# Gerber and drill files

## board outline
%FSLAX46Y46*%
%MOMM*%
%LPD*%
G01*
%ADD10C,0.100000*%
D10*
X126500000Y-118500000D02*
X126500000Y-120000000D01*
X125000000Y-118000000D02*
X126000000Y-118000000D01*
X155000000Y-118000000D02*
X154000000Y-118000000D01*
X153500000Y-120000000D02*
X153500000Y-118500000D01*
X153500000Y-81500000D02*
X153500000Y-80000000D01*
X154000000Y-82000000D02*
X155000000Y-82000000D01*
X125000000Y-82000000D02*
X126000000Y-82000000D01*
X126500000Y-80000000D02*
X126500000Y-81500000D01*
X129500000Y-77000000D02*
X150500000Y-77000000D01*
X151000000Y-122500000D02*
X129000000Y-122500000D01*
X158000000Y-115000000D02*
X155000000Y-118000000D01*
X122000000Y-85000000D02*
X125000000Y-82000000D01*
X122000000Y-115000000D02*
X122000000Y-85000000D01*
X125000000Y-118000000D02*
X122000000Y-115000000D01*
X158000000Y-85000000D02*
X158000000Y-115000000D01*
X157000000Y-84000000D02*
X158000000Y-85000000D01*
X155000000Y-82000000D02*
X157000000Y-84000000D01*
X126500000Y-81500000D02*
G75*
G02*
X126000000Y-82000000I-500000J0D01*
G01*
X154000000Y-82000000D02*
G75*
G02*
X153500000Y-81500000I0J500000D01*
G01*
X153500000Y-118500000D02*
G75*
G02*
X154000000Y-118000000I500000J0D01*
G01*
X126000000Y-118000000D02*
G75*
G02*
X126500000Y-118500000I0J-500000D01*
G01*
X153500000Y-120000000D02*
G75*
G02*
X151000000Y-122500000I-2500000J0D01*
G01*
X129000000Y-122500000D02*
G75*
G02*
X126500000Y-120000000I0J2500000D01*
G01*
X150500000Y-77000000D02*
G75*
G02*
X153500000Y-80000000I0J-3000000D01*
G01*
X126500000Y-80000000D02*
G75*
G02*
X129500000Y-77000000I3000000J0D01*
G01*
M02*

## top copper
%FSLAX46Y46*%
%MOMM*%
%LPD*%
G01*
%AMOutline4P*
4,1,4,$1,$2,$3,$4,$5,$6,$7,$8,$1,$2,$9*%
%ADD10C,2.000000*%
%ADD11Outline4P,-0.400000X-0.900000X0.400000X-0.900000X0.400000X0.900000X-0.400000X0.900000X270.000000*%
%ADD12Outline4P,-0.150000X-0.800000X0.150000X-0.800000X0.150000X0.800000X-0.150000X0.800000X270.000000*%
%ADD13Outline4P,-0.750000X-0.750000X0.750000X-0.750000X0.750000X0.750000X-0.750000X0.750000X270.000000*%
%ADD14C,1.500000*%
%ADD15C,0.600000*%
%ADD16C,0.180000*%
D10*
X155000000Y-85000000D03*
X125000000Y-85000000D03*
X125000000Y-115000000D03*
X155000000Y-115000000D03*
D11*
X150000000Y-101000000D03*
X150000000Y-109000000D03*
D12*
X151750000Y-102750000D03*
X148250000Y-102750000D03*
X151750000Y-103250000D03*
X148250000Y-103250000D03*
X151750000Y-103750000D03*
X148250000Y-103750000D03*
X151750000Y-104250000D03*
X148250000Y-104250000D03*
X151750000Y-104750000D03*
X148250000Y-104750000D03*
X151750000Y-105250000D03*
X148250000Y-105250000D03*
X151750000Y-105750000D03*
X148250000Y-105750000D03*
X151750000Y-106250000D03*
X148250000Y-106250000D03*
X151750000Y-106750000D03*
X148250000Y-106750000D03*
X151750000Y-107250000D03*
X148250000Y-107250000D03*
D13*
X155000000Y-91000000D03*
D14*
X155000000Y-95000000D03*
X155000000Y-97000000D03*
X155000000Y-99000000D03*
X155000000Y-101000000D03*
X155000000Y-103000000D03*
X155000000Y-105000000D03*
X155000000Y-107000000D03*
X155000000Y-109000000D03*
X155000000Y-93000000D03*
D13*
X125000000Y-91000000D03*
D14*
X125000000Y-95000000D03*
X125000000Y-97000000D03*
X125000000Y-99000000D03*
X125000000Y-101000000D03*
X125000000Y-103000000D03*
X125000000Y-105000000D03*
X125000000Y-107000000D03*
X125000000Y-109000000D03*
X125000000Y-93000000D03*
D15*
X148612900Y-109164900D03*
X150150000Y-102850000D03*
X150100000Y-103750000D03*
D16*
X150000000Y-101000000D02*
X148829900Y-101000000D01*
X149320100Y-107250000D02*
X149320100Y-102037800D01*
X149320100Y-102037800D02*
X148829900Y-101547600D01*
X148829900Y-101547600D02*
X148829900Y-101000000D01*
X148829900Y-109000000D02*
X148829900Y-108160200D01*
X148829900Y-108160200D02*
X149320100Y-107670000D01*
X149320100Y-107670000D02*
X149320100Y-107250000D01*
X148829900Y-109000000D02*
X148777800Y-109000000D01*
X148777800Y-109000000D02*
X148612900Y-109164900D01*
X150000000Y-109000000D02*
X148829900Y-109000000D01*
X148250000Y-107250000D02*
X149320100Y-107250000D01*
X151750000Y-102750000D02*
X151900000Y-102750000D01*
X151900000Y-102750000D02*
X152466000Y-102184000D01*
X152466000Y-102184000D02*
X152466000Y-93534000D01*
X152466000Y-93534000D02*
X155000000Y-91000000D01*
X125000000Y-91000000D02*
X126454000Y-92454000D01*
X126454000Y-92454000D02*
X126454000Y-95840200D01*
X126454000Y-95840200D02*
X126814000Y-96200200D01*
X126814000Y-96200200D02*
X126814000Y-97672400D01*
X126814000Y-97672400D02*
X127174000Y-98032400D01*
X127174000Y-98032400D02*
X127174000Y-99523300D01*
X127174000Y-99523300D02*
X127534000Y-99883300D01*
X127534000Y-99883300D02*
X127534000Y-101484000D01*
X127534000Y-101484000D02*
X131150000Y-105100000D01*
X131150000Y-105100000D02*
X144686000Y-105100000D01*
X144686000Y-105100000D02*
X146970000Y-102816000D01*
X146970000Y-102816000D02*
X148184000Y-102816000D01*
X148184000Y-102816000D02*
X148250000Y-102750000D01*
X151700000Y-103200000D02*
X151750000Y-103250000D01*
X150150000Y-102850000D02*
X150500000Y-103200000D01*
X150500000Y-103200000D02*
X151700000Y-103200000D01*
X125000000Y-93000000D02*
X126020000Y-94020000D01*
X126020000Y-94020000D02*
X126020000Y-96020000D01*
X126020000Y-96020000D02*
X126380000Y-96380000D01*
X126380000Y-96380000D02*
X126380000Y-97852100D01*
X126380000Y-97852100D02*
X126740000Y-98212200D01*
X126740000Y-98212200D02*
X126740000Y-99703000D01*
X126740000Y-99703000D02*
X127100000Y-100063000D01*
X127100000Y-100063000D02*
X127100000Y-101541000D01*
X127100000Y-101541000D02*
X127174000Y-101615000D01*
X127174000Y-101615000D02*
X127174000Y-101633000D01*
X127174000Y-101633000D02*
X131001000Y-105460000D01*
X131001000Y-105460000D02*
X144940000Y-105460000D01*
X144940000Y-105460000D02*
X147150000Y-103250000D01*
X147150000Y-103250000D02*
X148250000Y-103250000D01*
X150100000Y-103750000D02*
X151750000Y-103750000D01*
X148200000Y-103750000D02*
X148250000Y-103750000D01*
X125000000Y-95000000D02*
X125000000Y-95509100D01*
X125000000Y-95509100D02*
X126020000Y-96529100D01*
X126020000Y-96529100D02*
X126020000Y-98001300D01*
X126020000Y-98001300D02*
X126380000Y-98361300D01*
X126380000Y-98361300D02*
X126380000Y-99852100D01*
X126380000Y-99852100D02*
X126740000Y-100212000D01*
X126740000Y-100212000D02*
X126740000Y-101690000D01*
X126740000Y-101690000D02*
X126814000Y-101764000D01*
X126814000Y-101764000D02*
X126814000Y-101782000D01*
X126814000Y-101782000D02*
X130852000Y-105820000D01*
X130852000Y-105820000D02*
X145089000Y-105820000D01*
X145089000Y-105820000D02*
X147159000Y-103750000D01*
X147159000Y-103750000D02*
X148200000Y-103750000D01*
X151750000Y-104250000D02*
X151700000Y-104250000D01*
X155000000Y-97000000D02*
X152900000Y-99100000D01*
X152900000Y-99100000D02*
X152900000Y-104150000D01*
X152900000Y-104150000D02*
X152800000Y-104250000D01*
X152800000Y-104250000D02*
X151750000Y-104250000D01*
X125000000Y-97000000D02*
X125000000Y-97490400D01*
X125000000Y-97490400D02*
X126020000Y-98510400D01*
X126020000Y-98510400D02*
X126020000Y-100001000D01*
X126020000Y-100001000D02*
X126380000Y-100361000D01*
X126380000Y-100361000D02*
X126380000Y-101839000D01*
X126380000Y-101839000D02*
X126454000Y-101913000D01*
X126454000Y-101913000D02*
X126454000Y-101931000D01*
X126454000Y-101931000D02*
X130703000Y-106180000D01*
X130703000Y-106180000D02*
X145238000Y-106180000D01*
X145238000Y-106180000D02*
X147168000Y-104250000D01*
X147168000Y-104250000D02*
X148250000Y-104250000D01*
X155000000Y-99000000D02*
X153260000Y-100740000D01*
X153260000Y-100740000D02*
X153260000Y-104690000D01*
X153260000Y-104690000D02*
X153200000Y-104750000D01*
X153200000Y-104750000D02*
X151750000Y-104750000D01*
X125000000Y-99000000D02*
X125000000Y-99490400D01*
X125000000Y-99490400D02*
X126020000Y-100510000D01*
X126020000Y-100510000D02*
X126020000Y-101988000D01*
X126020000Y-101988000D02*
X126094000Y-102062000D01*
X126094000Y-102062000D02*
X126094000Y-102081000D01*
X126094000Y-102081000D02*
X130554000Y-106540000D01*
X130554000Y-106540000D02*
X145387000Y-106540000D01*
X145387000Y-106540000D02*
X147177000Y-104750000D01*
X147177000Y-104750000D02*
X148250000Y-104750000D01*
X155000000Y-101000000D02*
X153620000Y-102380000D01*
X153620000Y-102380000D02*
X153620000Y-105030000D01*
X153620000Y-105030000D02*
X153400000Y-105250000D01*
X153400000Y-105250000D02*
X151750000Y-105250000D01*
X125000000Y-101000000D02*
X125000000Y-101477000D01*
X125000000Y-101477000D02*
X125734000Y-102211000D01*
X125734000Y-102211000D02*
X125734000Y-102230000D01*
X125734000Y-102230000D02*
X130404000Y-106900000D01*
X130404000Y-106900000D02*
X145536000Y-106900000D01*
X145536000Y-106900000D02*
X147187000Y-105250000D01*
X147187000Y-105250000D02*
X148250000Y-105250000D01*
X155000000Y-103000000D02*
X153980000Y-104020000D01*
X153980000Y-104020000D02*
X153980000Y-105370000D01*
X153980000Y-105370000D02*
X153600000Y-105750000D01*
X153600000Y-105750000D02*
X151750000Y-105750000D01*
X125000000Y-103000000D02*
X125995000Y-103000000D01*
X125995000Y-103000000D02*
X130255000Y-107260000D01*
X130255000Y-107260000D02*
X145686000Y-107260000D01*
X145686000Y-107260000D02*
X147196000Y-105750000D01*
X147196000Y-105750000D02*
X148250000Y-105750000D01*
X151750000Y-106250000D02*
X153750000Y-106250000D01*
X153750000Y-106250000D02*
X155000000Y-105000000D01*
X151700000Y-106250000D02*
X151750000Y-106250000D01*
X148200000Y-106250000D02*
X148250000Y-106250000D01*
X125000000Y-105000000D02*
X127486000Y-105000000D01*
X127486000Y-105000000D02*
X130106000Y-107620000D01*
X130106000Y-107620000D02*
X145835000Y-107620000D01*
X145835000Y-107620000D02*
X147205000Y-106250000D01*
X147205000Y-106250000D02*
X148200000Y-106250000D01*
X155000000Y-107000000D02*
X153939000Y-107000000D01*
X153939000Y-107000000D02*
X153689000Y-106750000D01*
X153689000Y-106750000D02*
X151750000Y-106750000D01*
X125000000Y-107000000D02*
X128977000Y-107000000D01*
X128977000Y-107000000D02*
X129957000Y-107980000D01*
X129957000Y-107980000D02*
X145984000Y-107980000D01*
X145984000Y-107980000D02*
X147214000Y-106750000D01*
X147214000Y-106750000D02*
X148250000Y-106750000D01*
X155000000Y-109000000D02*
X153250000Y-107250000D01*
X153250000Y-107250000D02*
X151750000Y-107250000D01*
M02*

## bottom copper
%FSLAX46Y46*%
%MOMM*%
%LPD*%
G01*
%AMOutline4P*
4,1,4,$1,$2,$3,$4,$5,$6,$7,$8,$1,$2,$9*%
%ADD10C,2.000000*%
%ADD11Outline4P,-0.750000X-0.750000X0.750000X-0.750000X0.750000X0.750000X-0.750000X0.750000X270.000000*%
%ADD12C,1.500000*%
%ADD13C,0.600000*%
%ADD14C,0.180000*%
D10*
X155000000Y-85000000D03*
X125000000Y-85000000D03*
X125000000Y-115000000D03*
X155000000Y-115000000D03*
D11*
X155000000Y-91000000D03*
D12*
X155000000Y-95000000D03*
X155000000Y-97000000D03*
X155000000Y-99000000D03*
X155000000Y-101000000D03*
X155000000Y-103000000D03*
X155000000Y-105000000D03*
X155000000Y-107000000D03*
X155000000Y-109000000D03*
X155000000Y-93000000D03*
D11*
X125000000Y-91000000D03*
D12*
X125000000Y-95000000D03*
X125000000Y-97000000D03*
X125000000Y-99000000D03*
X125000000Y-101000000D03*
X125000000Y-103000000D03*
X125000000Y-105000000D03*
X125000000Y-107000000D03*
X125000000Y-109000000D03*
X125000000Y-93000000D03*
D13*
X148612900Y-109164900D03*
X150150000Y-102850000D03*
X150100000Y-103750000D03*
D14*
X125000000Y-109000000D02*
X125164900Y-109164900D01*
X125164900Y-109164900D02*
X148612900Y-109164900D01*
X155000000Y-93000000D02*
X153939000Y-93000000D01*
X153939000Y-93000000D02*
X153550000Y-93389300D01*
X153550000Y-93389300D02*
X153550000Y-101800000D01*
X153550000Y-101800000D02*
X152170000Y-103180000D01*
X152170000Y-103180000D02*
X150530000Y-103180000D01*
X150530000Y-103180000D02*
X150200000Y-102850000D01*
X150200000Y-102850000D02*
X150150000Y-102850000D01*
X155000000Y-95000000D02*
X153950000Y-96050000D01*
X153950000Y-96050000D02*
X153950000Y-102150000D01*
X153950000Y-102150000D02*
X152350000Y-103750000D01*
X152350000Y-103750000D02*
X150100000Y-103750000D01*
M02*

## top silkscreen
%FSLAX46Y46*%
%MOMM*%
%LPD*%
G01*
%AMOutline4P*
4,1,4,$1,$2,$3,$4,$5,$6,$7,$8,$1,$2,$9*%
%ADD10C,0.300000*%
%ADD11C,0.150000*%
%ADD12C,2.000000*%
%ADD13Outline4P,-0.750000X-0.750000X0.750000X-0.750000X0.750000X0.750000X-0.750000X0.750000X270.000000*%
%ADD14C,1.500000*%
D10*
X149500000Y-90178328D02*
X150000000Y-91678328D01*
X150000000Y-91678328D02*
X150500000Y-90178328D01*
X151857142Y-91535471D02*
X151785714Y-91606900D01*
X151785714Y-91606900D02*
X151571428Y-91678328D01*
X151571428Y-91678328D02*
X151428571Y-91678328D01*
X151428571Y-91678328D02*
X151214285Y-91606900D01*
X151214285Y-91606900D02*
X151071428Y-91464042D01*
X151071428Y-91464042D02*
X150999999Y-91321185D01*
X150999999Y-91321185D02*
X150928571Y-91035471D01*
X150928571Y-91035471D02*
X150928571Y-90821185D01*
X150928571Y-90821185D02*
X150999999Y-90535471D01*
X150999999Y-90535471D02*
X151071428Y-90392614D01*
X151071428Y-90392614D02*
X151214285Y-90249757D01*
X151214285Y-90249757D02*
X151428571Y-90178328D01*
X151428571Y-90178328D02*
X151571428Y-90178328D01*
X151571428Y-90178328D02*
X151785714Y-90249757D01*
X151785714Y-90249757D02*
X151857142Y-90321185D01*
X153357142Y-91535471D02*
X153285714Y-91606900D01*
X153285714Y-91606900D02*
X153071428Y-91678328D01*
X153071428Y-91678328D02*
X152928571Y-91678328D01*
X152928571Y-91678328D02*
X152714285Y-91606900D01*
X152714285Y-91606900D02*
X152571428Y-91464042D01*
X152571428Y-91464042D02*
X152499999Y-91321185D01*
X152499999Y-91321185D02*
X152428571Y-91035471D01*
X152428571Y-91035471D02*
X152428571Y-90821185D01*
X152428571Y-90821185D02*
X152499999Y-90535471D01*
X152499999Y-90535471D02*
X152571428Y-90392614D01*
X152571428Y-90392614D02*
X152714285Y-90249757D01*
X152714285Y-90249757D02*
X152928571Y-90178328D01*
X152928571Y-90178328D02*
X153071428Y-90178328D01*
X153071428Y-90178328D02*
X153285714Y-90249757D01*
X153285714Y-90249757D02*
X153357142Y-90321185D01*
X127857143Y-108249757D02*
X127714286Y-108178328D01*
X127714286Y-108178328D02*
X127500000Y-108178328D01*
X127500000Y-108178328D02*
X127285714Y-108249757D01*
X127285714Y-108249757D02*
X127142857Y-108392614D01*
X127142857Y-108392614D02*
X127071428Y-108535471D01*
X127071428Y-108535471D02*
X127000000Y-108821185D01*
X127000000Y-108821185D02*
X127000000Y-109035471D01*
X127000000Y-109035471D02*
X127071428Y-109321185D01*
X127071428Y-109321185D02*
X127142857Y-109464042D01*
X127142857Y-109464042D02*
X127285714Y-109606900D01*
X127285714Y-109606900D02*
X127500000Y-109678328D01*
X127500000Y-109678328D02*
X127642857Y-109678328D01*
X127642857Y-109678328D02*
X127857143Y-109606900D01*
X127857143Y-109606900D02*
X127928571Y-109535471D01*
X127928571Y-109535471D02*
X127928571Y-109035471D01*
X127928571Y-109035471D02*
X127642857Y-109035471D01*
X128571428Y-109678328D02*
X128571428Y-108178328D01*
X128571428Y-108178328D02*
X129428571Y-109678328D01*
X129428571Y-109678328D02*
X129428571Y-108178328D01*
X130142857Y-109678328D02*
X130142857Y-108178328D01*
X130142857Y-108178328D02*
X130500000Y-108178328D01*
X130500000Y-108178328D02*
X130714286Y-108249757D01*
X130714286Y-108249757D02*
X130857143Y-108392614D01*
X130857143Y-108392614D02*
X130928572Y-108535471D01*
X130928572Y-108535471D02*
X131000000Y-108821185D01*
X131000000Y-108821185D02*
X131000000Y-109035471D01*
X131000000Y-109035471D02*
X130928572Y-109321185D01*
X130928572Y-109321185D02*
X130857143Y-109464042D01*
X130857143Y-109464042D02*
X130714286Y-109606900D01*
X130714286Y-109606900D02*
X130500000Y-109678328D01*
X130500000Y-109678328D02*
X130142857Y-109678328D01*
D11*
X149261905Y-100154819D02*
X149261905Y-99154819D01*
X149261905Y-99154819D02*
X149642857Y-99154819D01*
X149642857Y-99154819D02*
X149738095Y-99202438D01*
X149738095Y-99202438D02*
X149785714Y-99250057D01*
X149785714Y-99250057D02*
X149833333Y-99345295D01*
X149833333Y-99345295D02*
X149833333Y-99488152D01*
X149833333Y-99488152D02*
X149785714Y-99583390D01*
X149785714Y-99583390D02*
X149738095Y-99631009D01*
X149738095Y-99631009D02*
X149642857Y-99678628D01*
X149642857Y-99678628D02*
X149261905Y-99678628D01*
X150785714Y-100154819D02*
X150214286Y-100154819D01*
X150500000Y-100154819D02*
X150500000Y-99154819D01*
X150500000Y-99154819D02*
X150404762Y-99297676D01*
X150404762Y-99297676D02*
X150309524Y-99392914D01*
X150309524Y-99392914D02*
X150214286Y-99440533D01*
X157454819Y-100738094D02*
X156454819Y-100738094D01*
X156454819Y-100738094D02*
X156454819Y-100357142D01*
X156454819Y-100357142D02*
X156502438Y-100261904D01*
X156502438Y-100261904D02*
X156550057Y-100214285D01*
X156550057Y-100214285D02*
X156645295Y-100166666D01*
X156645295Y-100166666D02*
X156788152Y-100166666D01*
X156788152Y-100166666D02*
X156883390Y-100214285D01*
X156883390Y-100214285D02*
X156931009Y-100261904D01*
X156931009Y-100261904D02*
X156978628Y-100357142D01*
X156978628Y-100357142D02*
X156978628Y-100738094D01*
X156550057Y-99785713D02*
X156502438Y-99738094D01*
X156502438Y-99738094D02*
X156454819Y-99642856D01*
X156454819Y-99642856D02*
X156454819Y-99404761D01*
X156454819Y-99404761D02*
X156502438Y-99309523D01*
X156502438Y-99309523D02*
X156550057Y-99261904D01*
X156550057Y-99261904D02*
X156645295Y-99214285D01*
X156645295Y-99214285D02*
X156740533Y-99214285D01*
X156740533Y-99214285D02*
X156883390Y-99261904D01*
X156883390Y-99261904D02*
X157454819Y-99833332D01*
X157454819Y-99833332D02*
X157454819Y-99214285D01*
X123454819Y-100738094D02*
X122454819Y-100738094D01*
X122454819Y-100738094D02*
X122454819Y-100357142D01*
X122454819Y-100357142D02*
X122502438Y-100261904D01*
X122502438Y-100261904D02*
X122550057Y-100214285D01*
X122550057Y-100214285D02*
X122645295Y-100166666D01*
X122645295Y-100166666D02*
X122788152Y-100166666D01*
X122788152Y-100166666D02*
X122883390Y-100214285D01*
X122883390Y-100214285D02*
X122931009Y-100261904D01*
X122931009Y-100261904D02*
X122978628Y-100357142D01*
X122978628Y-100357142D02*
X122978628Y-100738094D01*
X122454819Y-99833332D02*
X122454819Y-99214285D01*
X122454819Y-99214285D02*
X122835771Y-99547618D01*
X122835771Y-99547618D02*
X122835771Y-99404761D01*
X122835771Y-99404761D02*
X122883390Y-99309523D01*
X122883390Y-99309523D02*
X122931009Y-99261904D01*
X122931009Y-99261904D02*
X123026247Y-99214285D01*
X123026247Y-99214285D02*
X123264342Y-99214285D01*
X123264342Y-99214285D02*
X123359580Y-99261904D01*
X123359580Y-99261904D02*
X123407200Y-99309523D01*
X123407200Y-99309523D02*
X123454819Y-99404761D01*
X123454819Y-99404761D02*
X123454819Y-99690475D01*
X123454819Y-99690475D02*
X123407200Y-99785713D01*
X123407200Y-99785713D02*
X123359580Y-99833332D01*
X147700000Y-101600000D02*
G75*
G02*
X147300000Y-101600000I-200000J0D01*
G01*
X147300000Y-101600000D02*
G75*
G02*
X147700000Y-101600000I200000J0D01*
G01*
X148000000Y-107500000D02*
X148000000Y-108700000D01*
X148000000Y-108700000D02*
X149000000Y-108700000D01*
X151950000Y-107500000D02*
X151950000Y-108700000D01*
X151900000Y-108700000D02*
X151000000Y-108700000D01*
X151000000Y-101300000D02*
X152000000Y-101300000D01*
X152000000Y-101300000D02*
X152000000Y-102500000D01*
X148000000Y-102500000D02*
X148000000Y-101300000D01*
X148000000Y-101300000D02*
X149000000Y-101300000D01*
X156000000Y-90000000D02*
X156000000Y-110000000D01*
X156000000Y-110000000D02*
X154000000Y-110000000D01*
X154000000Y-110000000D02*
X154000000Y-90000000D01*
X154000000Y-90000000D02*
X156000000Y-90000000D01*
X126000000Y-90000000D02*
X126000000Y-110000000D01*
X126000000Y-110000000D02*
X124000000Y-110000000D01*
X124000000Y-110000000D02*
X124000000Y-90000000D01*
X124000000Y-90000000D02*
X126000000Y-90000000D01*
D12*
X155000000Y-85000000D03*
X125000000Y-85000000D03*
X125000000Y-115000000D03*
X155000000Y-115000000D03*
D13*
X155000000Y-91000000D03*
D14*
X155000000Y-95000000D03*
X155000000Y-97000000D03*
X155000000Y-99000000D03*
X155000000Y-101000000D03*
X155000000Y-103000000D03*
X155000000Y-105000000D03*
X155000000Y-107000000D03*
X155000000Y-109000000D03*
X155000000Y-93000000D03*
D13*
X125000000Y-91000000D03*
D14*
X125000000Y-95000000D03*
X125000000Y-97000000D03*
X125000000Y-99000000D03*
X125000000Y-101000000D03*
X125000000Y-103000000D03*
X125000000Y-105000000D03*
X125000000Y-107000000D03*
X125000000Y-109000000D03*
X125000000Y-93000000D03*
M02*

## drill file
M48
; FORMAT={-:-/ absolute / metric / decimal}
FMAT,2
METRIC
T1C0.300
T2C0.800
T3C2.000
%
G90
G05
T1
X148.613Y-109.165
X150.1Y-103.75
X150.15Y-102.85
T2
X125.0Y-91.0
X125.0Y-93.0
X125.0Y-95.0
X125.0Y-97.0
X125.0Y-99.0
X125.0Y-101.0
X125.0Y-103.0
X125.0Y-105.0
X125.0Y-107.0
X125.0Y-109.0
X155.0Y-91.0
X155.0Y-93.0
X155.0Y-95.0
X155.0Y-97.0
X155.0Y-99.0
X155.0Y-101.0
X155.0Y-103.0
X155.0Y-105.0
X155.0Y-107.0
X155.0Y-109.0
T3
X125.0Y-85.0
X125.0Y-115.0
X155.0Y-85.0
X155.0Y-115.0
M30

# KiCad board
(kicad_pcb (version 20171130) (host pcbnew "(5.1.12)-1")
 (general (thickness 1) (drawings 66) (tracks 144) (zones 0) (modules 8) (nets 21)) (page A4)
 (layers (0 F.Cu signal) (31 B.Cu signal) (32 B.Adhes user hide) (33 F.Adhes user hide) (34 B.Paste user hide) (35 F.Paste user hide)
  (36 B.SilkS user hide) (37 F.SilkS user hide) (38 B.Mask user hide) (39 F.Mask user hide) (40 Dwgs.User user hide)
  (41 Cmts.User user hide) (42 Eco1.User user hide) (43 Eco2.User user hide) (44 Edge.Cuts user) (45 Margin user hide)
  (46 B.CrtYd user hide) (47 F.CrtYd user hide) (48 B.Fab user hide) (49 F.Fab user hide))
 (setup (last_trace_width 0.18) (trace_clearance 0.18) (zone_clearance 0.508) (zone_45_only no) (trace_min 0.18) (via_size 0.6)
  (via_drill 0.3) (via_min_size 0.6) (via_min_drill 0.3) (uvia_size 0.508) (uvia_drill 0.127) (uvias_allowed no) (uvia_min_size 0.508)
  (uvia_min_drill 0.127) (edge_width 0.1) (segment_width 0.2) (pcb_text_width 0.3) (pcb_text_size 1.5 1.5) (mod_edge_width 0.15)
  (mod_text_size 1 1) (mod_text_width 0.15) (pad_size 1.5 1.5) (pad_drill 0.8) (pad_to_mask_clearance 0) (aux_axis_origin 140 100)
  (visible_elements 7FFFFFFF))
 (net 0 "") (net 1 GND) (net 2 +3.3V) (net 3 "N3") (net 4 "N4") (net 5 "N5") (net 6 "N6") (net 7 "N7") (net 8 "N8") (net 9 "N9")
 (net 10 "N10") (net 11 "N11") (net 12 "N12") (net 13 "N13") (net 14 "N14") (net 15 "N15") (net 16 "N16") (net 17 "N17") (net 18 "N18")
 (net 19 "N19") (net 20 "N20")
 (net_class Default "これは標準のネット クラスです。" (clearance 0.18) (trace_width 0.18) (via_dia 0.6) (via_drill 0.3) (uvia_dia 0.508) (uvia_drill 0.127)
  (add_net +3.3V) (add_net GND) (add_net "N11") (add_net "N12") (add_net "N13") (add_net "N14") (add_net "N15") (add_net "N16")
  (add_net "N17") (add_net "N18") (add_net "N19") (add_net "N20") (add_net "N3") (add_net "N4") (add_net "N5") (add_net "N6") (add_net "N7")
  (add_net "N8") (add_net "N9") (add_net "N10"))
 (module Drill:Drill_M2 (layer F.Cu) (at 155 85)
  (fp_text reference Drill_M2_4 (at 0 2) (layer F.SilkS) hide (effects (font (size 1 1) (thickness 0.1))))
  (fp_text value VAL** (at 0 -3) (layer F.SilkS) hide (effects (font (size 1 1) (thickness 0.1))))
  (pad "" thru_hole circle (at 0 0) (size 2 2) (drill 2) (layers *.Cu *.Mask F.SilkS)))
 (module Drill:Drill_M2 (layer F.Cu) (at 125 85)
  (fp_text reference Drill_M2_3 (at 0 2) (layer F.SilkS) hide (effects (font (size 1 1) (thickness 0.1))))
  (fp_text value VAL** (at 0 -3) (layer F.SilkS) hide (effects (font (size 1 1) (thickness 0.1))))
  (pad "" thru_hole circle (at 0 0) (size 2 2) (drill 2) (layers *.Cu *.Mask F.SilkS)))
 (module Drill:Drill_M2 (layer F.Cu) (at 125 115)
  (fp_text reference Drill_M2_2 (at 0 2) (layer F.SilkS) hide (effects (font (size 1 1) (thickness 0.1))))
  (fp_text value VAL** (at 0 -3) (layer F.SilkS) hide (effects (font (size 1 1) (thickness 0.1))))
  (pad "" thru_hole circle (at 0 0) (size 2 2) (drill 2) (layers *.Cu *.Mask F.SilkS)))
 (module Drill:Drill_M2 (layer F.Cu) (at 155 115)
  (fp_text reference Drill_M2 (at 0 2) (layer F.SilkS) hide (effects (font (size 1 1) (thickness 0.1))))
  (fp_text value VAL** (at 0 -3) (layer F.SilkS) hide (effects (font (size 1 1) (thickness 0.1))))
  (pad "" thru_hole circle (at 0 0) (size 2 2) (drill 2) (layers *.Cu *.Mask F.SilkS)))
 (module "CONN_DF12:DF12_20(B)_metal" (layer F.Cu) (at 150 105)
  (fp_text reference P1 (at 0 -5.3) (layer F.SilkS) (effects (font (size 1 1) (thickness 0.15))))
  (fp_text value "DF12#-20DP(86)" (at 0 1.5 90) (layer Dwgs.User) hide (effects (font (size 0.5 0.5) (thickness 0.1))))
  (fp_circle (center -2.5 -3.4) (end -2.5 -3.2) (layer F.SilkS) (width 0.15))
  (fp_line (start -2 2.5) (end -2 3.7) (layer F.SilkS) (width 0.15))
  (fp_line (start -2 3.7) (end -1 3.7) (layer F.SilkS) (width 0.15))
  (fp_line (start 1.95 2.5) (end 1.95 3.7) (layer F.SilkS) (width 0.15))
  (fp_line (start 1.9 3.7) (end 1 3.7) (layer F.SilkS) (width 0.15))
  (fp_line (start 1 -3.7) (end 2 -3.7) (layer F.SilkS) (width 0.15))
  (fp_line (start 2 -3.7) (end 2 -2.5) (layer F.SilkS) (width 0.15))
  (fp_line (start -2 -2.5) (end -2 -3.7) (layer F.SilkS) (width 0.15))
  (fp_line (start -2 -3.7) (end -1 -3.7) (layer F.SilkS) (width 0.15))
  (pad 21 smd trapezoid (at 0 -4 270) (size 0.8 1.8) (layers F.Cu F.Paste F.Mask) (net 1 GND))
  (pad 22 smd trapezoid (at 0 4 270) (size 0.8 1.8) (layers F.Cu F.Paste F.Mask) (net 1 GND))
  (pad 1 smd trapezoid (at 1.75 -2.25 270) (size 0.3 1.6) (layers F.Cu F.Paste F.Mask) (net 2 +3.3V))
  (pad 2 smd trapezoid (at -1.75 -2.25 270) (size 0.3 1.6) (layers F.Cu F.Paste F.Mask) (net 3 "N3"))
  (pad 3 smd trapezoid (at 1.75 -1.75 270) (size 0.3 1.6) (layers F.Cu F.Paste F.Mask) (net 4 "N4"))
  (pad 4 smd trapezoid (at -1.75 -1.75 270) (size 0.3 1.6) (layers F.Cu F.Paste F.Mask) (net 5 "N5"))
  (pad 5 smd trapezoid (at 1.75 -1.25 270) (size 0.3 1.6) (layers F.Cu F.Paste F.Mask) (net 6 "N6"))
  (pad 6 smd trapezoid (at -1.75 -1.25 270) (size 0.3 1.6) (layers F.Cu F.Paste F.Mask) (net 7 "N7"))
  (pad 7 smd trapezoid (at 1.75 -0.75 270) (size 0.3 1.6) (layers F.Cu F.Paste F.Mask) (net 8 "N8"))
  (pad 8 smd trapezoid (at -1.75 -0.75 270) (size 0.3 1.6) (layers F.Cu F.Paste F.Mask) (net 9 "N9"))
  (pad 9 smd trapezoid (at 1.75 -0.25 270) (size 0.3 1.6) (layers F.Cu F.Paste F.Mask) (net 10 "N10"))
  (pad 10 smd trapezoid (at -1.75 -0.25 270) (size 0.3 1.6) (layers F.Cu F.Paste F.Mask) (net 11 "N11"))
  (pad 11 smd trapezoid (at 1.75 0.25 270) (size 0.3 1.6) (layers F.Cu F.Paste F.Mask) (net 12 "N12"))
  (pad 12 smd trapezoid (at -1.75 0.25 270) (size 0.3 1.6) (layers F.Cu F.Paste F.Mask) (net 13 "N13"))
  (pad 13 smd trapezoid (at 1.75 0.75 270) (size 0.3 1.6) (layers F.Cu F.Paste F.Mask) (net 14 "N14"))
  (pad 14 smd trapezoid (at -1.75 0.75 270) (size 0.3 1.6) (layers F.Cu F.Paste F.Mask) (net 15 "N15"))
  (pad 15 smd trapezoid (at 1.75 1.25 270) (size 0.3 1.6) (layers F.Cu F.Paste F.Mask) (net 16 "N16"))
  (pad 16 smd trapezoid (at -1.75 1.25 270) (size 0.3 1.6) (layers F.Cu F.Paste F.Mask) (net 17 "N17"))
  (pad 17 smd trapezoid (at 1.75 1.75 270) (size 0.3 1.6) (layers F.Cu F.Paste F.Mask) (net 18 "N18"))
  (pad 18 smd trapezoid (at -1.75 1.75 270) (size 0.3 1.6) (layers F.Cu F.Paste F.Mask) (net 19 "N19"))
  (pad 19 smd trapezoid (at 1.75 2.25 270) (size 0.3 1.6) (layers F.Cu F.Paste F.Mask) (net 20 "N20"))
  (pad 20 smd trapezoid (at -1.75 2.25 270) (size 0.3 1.6) (layers F.Cu F.Paste F.Mask) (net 1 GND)))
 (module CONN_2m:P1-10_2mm (layer F.Cu) (at 155 100 270)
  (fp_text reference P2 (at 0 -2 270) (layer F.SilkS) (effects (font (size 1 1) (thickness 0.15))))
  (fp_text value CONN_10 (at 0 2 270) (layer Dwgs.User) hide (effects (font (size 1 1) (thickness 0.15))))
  (fp_line (start -10 -1) (end 10 -1) (layer F.SilkS) (width 0.15))
  (fp_line (start 10 -1) (end 10 1) (layer F.SilkS) (width 0.15))
  (fp_line (start 10 1) (end -10 1) (layer F.SilkS) (width 0.15))
  (fp_line (start -10 1) (end -10 -1) (layer F.SilkS) (width 0.15))
  (pad 1 thru_hole trapezoid (at -9 0 270) (size 1.5 1.5) (drill 0.8) (layers *.Cu *.Mask F.SilkS) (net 2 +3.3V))
  (pad 3 thru_hole circle (at -5 0 270) (size 1.5 1.5) (drill 0.8) (layers *.Cu *.Mask F.SilkS) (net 6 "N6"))
  (pad 4 thru_hole circle (at -3 0 270) (size 1.5 1.5) (drill 0.8) (layers *.Cu *.Mask F.SilkS) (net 8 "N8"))
  (pad 5 thru_hole circle (at -1 0 270) (size 1.5 1.5) (drill 0.8) (layers *.Cu *.Mask F.SilkS) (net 10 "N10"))
  (pad 6 thru_hole circle (at 1 0 270) (size 1.5 1.5) (drill 0.8) (layers *.Cu *.Mask F.SilkS) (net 12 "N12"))
  (pad 7 thru_hole circle (at 3 0 270) (size 1.5 1.5) (drill 0.8) (layers *.Cu *.Mask F.SilkS) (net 14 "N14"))
  (pad 8 thru_hole circle (at 5 0 270) (size 1.5 1.5) (drill 0.8) (layers *.Cu *.Mask F.SilkS) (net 16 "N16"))
  (pad 9 thru_hole circle (at 7 0 270) (size 1.5 1.5) (drill 0.8) (layers *.Cu *.Mask F.SilkS) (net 18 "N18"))
  (pad 10 thru_hole circle (at 9 0 270) (size 1.5 1.5) (drill 0.8) (layers *.Cu *.Mask F.SilkS) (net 20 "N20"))
  (pad 2 thru_hole circle (at -7 0 270) (size 1.5 1.5) (drill 0.8) (layers *.Cu *.Mask F.SilkS) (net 4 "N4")))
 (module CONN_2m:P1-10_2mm (layer F.Cu) (at 125 100 270)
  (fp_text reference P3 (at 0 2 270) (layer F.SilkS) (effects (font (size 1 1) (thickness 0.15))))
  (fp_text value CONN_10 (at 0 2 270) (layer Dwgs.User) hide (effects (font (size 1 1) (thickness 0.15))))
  (fp_line (start -10 -1) (end 10 -1) (layer F.SilkS) (width 0.15))
  (fp_line (start 10 -1) (end 10 1) (layer F.SilkS) (width 0.15))
  (fp_line (start 10 1) (end -10 1) (layer F.SilkS) (width 0.15))
  (fp_line (start -10 1) (end -10 -1) (layer F.SilkS) (width 0.15))
  (pad 1 thru_hole trapezoid (at -9 0 270) (size 1.5 1.5) (drill 0.8) (layers *.Cu *.Mask F.SilkS) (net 3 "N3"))
  (pad 3 thru_hole circle (at -5 0 270) (size 1.5 1.5) (drill 0.8) (layers *.Cu *.Mask F.SilkS) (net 7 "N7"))
  (pad 4 thru_hole circle (at -3 0 270) (size 1.5 1.5) (drill 0.8) (layers *.Cu *.Mask F.SilkS) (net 9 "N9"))
  (pad 5 thru_hole circle (at -1 0 270) (size 1.5 1.5) (drill 0.8) (layers *.Cu *.Mask F.SilkS) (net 11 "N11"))
  (pad 6 thru_hole circle (at 1 0 270) (size 1.5 1.5) (drill 0.8) (layers *.Cu *.Mask F.SilkS) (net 13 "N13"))
  (pad 7 thru_hole circle (at 3 0 270) (size 1.5 1.5) (drill 0.8) (layers *.Cu *.Mask F.SilkS) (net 15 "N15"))
  (pad 8 thru_hole circle (at 5 0 270) (size 1.5 1.5) (drill 0.8) (layers *.Cu *.Mask F.SilkS) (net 17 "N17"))
  (pad 9 thru_hole circle (at 7 0 270) (size 1.5 1.5) (drill 0.8) (layers *.Cu *.Mask F.SilkS) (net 19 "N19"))
  (pad 10 thru_hole circle (at 9 0 270) (size 1.5 1.5) (drill 0.8) (layers *.Cu *.Mask F.SilkS) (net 1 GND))
  (pad 2 thru_hole circle (at -7 0 270) (size 1.5 1.5) (drill 0.8) (layers *.Cu *.Mask F.SilkS) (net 5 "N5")))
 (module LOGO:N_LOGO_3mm (layer B.Cu) (at 140 95)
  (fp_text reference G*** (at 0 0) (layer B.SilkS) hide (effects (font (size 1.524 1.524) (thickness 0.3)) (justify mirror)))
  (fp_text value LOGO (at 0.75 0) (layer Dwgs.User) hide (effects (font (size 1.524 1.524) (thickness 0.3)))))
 (gr_line (start 126.5 118.5) (end 126.5 120) (angle 90) (layer Edge.Cuts) (width 0.1))
 (gr_line (start 125 118) (end 126 118) (angle 90) (layer Edge.Cuts) (width 0.1))
 (gr_line (start 155 118) (end 154 118) (angle 90) (layer Edge.Cuts) (width 0.1))
 (gr_line (start 153.5 120) (end 153.5 118.5) (angle 90) (layer Edge.Cuts) (width 0.1))
 (gr_line (start 153.5 81.5) (end 153.5 80) (angle 90) (layer Edge.Cuts) (width 0.1))
 (gr_line (start 154 82) (end 155 82) (angle 90) (layer Edge.Cuts) (width 0.1))
 (gr_line (start 125 82) (end 126 82) (angle 90) (layer Edge.Cuts) (width 0.1))
 (gr_line (start 126.5 80) (end 126.5 81.5) (angle 90) (layer Edge.Cuts) (width 0.1))
 (gr_line (start 129.5 77) (end 150.5 77) (angle 90) (layer Edge.Cuts) (width 0.1))
 (gr_line (start 151 122.5) (end 129 122.5) (angle 90) (layer Edge.Cuts) (width 0.1))
 (gr_line (start 158 115) (end 155 118) (angle 90) (layer Edge.Cuts) (width 0.1))
 (gr_line (start 122 85) (end 125 82) (angle 90) (layer Edge.Cuts) (width 0.1))
 (gr_line (start 122 115) (end 122 85) (angle 90) (layer Edge.Cuts) (width 0.1))
 (gr_line (start 125 118) (end 122 115) (angle 90) (layer Edge.Cuts) (width 0.1))
 (gr_line (start 158 85) (end 158 115) (angle 90) (layer Edge.Cuts) (width 0.1))
 (gr_line (start 157 84) (end 158 85) (angle 90) (layer Edge.Cuts) (width 0.1))
 (gr_line (start 155 82) (end 157 84) (angle 90) (layer Edge.Cuts) (width 0.1))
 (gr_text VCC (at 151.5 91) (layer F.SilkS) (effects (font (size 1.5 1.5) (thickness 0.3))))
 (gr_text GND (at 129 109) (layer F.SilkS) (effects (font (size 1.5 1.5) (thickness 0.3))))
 (gr_arc (start 126 81.5) (end 126.5 81.5) (angle 90) (layer Edge.Cuts) (width 0.1))
 (gr_arc (start 154 81.5) (end 154 82) (angle 90) (layer Edge.Cuts) (width 0.1))
 (gr_arc (start 154 118.5) (end 153.5 118.5) (angle 90) (layer Edge.Cuts) (width 0.1))
 (gr_arc (start 126 118.5) (end 126 118) (angle 90) (layer Edge.Cuts) (width 0.1))
 (gr_arc (start 151 120) (end 153.5 120) (angle 90) (layer Edge.Cuts) (width 0.1))
 (gr_arc (start 129 120) (end 129 122.5) (angle 90) (layer Edge.Cuts) (width 0.1))
 (gr_arc (start 150.5 80) (end 150.5 77) (angle 90) (layer Edge.Cuts) (width 0.1))
 (gr_arc (start 129.5 80) (end 126.5 80) (angle 90) (layer Edge.Cuts) (width 0.1))
 (segment (start 150 101) (end 148.8299 101) (width 0.18) (layer F.Cu) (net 1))
 (segment (start 149.3201 107.25) (end 149.3201 102.0378) (width 0.18) (layer F.Cu) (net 1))
 (segment (start 149.3201 102.0378) (end 148.8299 101.5476) (width 0.18) (layer F.Cu) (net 1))
 (segment (start 148.8299 101.5476) (end 148.8299 101) (width 0.18) (layer F.Cu) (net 1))
 (segment (start 148.8299 109) (end 148.8299 108.1602) (width 0.18) (layer F.Cu) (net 1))
 (segment (start 148.8299 108.1602) (end 149.3201 107.67) (width 0.18) (layer F.Cu) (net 1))
 (segment (start 149.3201 107.67) (end 149.3201 107.25) (width 0.18) (layer F.Cu) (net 1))
 (segment (start 148.8299 109) (end 148.7778 109) (width 0.18) (layer F.Cu) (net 1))
 (segment (start 148.7778 109) (end 148.6129 109.1649) (width 0.18) (layer F.Cu) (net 1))
 (segment (start 125 109) (end 125.1649 109.1649) (width 0.18) (layer B.Cu) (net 1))
 (segment (start 125.1649 109.1649) (end 148.6129 109.1649) (width 0.18) (layer B.Cu) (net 1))
 (segment (start 150 109) (end 148.8299 109) (width 0.18) (layer F.Cu) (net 1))
 (segment (start 148.25 107.25) (end 149.3201 107.25) (width 0.18) (layer F.Cu) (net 1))
 (via (at 148.6129 109.1649) (size 0.6) (layers F.Cu B.Cu) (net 1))
 (segment (start 151.75 102.75) (end 151.9 102.75) (width 0.18) (layer F.Cu) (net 2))
 (segment (start 151.9 102.75) (end 152.466 102.184) (width 0.18) (layer F.Cu) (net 2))
 (segment (start 152.466 102.184) (end 152.466 93.534) (width 0.18) (layer F.Cu) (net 2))
 (segment (start 152.466 93.534) (end 155 91) (width 0.18) (layer F.Cu) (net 2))
 (segment (start 125 91) (end 126.454 92.454) (width 0.18) (layer F.Cu) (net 3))
 (segment (start 126.454 92.454) (end 126.454 95.8402) (width 0.18) (layer F.Cu) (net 3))
 (segment (start 126.454 95.8402) (end 126.814 96.2002) (width 0.18) (layer F.Cu) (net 3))
 (segment (start 126.814 96.2002) (end 126.814 97.6724) (width 0.18) (layer F.Cu) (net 3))
 (segment (start 126.814 97.6724) (end 127.174 98.0324) (width 0.18) (layer F.Cu) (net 3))
 (segment (start 127.174 98.0324) (end 127.174 99.5233) (width 0.18) (layer F.Cu) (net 3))
 (segment (start 127.174 99.5233) (end 127.534 99.8833) (width 0.18) (layer F.Cu) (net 3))
 (segment (start 127.534 99.8833) (end 127.534 101.484) (width 0.18) (layer F.Cu) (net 3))
 (segment (start 127.534 101.484) (end 131.15 105.1) (width 0.18) (layer F.Cu) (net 3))
 (segment (start 131.15 105.1) (end 144.686 105.1) (width 0.18) (layer F.Cu) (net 3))
 (segment (start 144.686 105.1) (end 146.97 102.816) (width 0.18) (layer F.Cu) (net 3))
 (segment (start 146.97 102.816) (end 148.184 102.816) (width 0.18) (layer F.Cu) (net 3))
 (segment (start 148.184 102.816) (end 148.25 102.75) (width 0.18) (layer F.Cu) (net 3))
 (segment (start 151.7 103.2) (end 151.75 103.25) (width 0.18) (layer F.Cu) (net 4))
 (segment (start 150.15 102.85) (end 150.5 103.2) (width 0.18) (layer F.Cu) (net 4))
 (segment (start 150.5 103.2) (end 151.7 103.2) (width 0.18) (layer F.Cu) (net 4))
 (segment (start 155 93) (end 153.939 93) (width 0.18) (layer B.Cu) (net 4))
 (segment (start 153.939 93) (end 153.55 93.3893) (width 0.18) (layer B.Cu) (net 4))
 (segment (start 153.55 93.3893) (end 153.55 101.8) (width 0.18) (layer B.Cu) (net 4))
 (segment (start 153.55 101.8) (end 152.17 103.18) (width 0.18) (layer B.Cu) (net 4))
 (segment (start 152.17 103.18) (end 150.53 103.18) (width 0.18) (layer B.Cu) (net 4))
 (segment (start 150.53 103.18) (end 150.2 102.85) (width 0.18) (layer B.Cu) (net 4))
 (segment (start 150.2 102.85) (end 150.15 102.85) (width 0.18) (layer B.Cu) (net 4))
 (via (at 150.15 102.85) (size 0.6) (layers F.Cu B.Cu) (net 4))
 (segment (start 125 93) (end 126.02 94.02) (width 0.18) (layer F.Cu) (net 5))
 (segment (start 126.02 94.02) (end 126.02 96.02) (width 0.18) (layer F.Cu) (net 5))
 (segment (start 126.02 96.02) (end 126.38 96.38) (width 0.18) (layer F.Cu) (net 5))
 (segment (start 126.38 96.38) (end 126.38 97.8521) (width 0.18) (layer F.Cu) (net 5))
 (segment (start 126.38 97.8521) (end 126.74 98.2122) (width 0.18) (layer F.Cu) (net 5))
 (segment (start 126.74 98.2122) (end 126.74 99.703) (width 0.18) (layer F.Cu) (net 5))
 (segment (start 126.74 99.703) (end 127.1 100.063) (width 0.18) (layer F.Cu) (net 5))
 (segment (start 127.1 100.063) (end 127.1 101.541) (width 0.18) (layer F.Cu) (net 5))
 (segment (start 127.1 101.541) (end 127.174 101.615) (width 0.18) (layer F.Cu) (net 5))
 (segment (start 127.174 101.615) (end 127.174 101.633) (width 0.18) (layer F.Cu) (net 5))
 (segment (start 127.174 101.633) (end 131.001 105.46) (width 0.18) (layer F.Cu) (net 5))
 (segment (start 131.001 105.46) (end 144.94 105.46) (width 0.18) (layer F.Cu) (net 5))
 (segment (start 144.94 105.46) (end 147.15 103.25) (width 0.18) (layer F.Cu) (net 5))
 (segment (start 147.15 103.25) (end 148.25 103.25) (width 0.18) (layer F.Cu) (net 5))
 (segment (start 150.1 103.75) (end 151.75 103.75) (width 0.18) (layer F.Cu) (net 6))
 (segment (start 155 95) (end 153.95 96.05) (width 0.18) (layer B.Cu) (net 6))
 (segment (start 153.95 96.05) (end 153.95 102.15) (width 0.18) (layer B.Cu) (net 6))
 (segment (start 153.95 102.15) (end 152.35 103.75) (width 0.18) (layer B.Cu) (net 6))
 (segment (start 152.35 103.75) (end 150.1 103.75) (width 0.18) (layer B.Cu) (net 6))
 (via (at 150.1 103.75) (size 0.6) (layers F.Cu B.Cu) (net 6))
 (segment (start 148.2 103.75) (end 148.25 103.75) (width 0.18) (layer F.Cu) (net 7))
 (segment (start 125 95) (end 125 95.5091) (width 0.18) (layer F.Cu) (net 7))
 (segment (start 125 95.5091) (end 126.02 96.5291) (width 0.18) (layer F.Cu) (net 7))
 (segment (start 126.02 96.5291) (end 126.02 98.0013) (width 0.18) (layer F.Cu) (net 7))
 (segment (start 126.02 98.0013) (end 126.38 98.3613) (width 0.18) (layer F.Cu) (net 7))
 (segment (start 126.38 98.3613) (end 126.38 99.8521) (width 0.18) (layer F.Cu) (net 7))
 (segment (start 126.38 99.8521) (end 126.74 100.212) (width 0.18) (layer F.Cu) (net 7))
 (segment (start 126.74 100.212) (end 126.74 101.69) (width 0.18) (layer F.Cu) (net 7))
 (segment (start 126.74 101.69) (end 126.814 101.764) (width 0.18) (layer F.Cu) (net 7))
 (segment (start 126.814 101.764) (end 126.814 101.782) (width 0.18) (layer F.Cu) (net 7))
 (segment (start 126.814 101.782) (end 130.852 105.82) (width 0.18) (layer F.Cu) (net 7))
 (segment (start 130.852 105.82) (end 145.089 105.82) (width 0.18) (layer F.Cu) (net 7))
 (segment (start 145.089 105.82) (end 147.159 103.75) (width 0.18) (layer F.Cu) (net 7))
 (segment (start 147.159 103.75) (end 148.2 103.75) (width 0.18) (layer F.Cu) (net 7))
 (segment (start 151.75 104.25) (end 151.7 104.25) (width 0.18) (layer F.Cu) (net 8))
 (segment (start 155 97) (end 152.9 99.1) (width 0.18) (layer F.Cu) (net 8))
 (segment (start 152.9 99.1) (end 152.9 104.15) (width 0.18) (layer F.Cu) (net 8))
 (segment (start 152.9 104.15) (end 152.8 104.25) (width 0.18) (layer F.Cu) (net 8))
 (segment (start 152.8 104.25) (end 151.75 104.25) (width 0.18) (layer F.Cu) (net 8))
 (segment (start 125 97) (end 125 97.4904) (width 0.18) (layer F.Cu) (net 9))
 (segment (start 125 97.4904) (end 126.02 98.5104) (width 0.18) (layer F.Cu) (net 9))
 (segment (start 126.02 98.5104) (end 126.02 100.001) (width 0.18) (layer F.Cu) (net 9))
 (segment (start 126.02 100.001) (end 126.38 100.361) (width 0.18) (layer F.Cu) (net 9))
 (segment (start 126.38 100.361) (end 126.38 101.839) (width 0.18) (layer F.Cu) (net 9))
 (segment (start 126.38 101.839) (end 126.454 101.913) (width 0.18) (layer F.Cu) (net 9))
 (segment (start 126.454 101.913) (end 126.454 101.931) (width 0.18) (layer F.Cu) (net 9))
 (segment (start 126.454 101.931) (end 130.703 106.18) (width 0.18) (layer F.Cu) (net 9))
 (segment (start 130.703 106.18) (end 145.238 106.18) (width 0.18) (layer F.Cu) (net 9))
 (segment (start 145.238 106.18) (end 147.168 104.25) (width 0.18) (layer F.Cu) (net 9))
 (segment (start 147.168 104.25) (end 148.25 104.25) (width 0.18) (layer F.Cu) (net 9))
 (segment (start 155 99) (end 153.26 100.74) (width 0.18) (layer F.Cu) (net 10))
 (segment (start 153.26 100.74) (end 153.26 104.69) (width 0.18) (layer F.Cu) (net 10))
 (segment (start 153.26 104.69) (end 153.2 104.75) (width 0.18) (layer F.Cu) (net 10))
 (segment (start 153.2 104.75) (end 151.75 104.75) (width 0.18) (layer F.Cu) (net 10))
 (segment (start 125 99) (end 125 99.4904) (width 0.18) (layer F.Cu) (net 11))
 (segment (start 125 99.4904) (end 126.02 100.51) (width 0.18) (layer F.Cu) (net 11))
 (segment (start 126.02 100.51) (end 126.02 101.988) (width 0.18) (layer F.Cu) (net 11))
 (segment (start 126.02 101.988) (end 126.094 102.062) (width 0.18) (layer F.Cu) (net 11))
 (segment (start 126.094 102.062) (end 126.094 102.081) (width 0.18) (layer F.Cu) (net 11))
 (segment (start 126.094 102.081) (end 130.554 106.54) (width 0.18) (layer F.Cu) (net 11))
 (segment (start 130.554 106.54) (end 145.387 106.54) (width 0.18) (layer F.Cu) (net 11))
 (segment (start 145.387 106.54) (end 147.177 104.75) (width 0.18) (layer F.Cu) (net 11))
 (segment (start 147.177 104.75) (end 148.25 104.75) (width 0.18) (layer F.Cu) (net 11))
 (segment (start 155 101) (end 153.62 102.38) (width 0.18) (layer F.Cu) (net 12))
 (segment (start 153.62 102.38) (end 153.62 105.03) (width 0.18) (layer F.Cu) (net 12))
 (segment (start 153.62 105.03) (end 153.4 105.25) (width 0.18) (layer F.Cu) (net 12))
 (segment (start 153.4 105.25) (end 151.75 105.25) (width 0.18) (layer F.Cu) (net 12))
 (segment (start 125 101) (end 125 101.477) (width 0.18) (layer F.Cu) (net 13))
 (segment (start 125 101.477) (end 125.734 102.211) (width 0.18) (layer F.Cu) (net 13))
 (segment (start 125.734 102.211) (end 125.734 102.23) (width 0.18) (layer F.Cu) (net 13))
 (segment (start 125.734 102.23) (end 130.404 106.9) (width 0.18) (layer F.Cu) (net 13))
 (segment (start 130.404 106.9) (end 145.536 106.9) (width 0.18) (layer F.Cu) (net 13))
 (segment (start 145.536 106.9) (end 147.187 105.25) (width 0.18) (layer F.Cu) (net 13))
 (segment (start 147.187 105.25) (end 148.25 105.25) (width 0.18) (layer F.Cu) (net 13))
 (segment (start 155 103) (end 153.98 104.02) (width 0.18) (layer F.Cu) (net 14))
 (segment (start 153.98 104.02) (end 153.98 105.37) (width 0.18) (layer F.Cu) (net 14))
 (segment (start 153.98 105.37) (end 153.6 105.75) (width 0.18) (layer F.Cu) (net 14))
 (segment (start 153.6 105.75) (end 151.75 105.75) (width 0.18) (layer F.Cu) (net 14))
 (segment (start 125 103) (end 125.995 103) (width 0.18) (layer F.Cu) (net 15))
 (segment (start 125.995 103) (end 130.255 107.26) (width 0.18) (layer F.Cu) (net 15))
 (segment (start 130.255 107.26) (end 145.686 107.26) (width 0.18) (layer F.Cu) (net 15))
 (segment (start 145.686 107.26) (end 147.196 105.75) (width 0.18) (layer F.Cu) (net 15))
 (segment (start 147.196 105.75) (end 148.25 105.75) (width 0.18) (layer F.Cu) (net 15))
 (segment (start 151.75 106.25) (end 153.75 106.25) (width 0.18) (layer F.Cu) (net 16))
 (segment (start 153.75 106.25) (end 155 105) (width 0.18) (layer F.Cu) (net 16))
 (segment (start 151.7 106.25) (end 151.75 106.25) (width 0.18) (layer F.Cu) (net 16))
 (segment (start 148.2 106.25) (end 148.25 106.25) (width 0.18) (layer F.Cu) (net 17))
 (segment (start 125 105) (end 127.486 105) (width 0.18) (layer F.Cu) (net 17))
 (segment (start 127.486 105) (end 130.106 107.62) (width 0.18) (layer F.Cu) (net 17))
 (segment (start 130.106 107.62) (end 145.835 107.62) (width 0.18) (layer F.Cu) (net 17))
 (segment (start 145.835 107.62) (end 147.205 106.25) (width 0.18) (layer F.Cu) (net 17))
 (segment (start 147.205 106.25) (end 148.2 106.25) (width 0.18) (layer F.Cu) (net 17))
 (segment (start 155 107) (end 153.939 107) (width 0.18) (layer F.Cu) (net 18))
 (segment (start 153.939 107) (end 153.689 106.75) (width 0.18) (layer F.Cu) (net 18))
 (segment (start 153.689 106.75) (end 151.75 106.75) (width 0.18) (layer F.Cu) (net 18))
 (segment (start 125 107) (end 128.977 107) (width 0.18) (layer F.Cu) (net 19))
 (segment (start 128.977 107) (end 129.957 107.98) (width 0.18) (layer F.Cu) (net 19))
 (segment (start 129.957 107.98) (end 145.984 107.98) (width 0.18) (layer F.Cu) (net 19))
 (segment (start 145.984 107.98) (end 147.214 106.75) (width 0.18) (layer F.Cu) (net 19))
 (segment (start 147.214 106.75) (end 148.25 106.75) (width 0.18) (layer F.Cu) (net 19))
 (segment (start 155 109) (end 153.25 107.25) (width 0.18) (layer F.Cu) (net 20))
 (segment (start 153.25 107.25) (end 151.75 107.25) (width 0.18) (layer F.Cu) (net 20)))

